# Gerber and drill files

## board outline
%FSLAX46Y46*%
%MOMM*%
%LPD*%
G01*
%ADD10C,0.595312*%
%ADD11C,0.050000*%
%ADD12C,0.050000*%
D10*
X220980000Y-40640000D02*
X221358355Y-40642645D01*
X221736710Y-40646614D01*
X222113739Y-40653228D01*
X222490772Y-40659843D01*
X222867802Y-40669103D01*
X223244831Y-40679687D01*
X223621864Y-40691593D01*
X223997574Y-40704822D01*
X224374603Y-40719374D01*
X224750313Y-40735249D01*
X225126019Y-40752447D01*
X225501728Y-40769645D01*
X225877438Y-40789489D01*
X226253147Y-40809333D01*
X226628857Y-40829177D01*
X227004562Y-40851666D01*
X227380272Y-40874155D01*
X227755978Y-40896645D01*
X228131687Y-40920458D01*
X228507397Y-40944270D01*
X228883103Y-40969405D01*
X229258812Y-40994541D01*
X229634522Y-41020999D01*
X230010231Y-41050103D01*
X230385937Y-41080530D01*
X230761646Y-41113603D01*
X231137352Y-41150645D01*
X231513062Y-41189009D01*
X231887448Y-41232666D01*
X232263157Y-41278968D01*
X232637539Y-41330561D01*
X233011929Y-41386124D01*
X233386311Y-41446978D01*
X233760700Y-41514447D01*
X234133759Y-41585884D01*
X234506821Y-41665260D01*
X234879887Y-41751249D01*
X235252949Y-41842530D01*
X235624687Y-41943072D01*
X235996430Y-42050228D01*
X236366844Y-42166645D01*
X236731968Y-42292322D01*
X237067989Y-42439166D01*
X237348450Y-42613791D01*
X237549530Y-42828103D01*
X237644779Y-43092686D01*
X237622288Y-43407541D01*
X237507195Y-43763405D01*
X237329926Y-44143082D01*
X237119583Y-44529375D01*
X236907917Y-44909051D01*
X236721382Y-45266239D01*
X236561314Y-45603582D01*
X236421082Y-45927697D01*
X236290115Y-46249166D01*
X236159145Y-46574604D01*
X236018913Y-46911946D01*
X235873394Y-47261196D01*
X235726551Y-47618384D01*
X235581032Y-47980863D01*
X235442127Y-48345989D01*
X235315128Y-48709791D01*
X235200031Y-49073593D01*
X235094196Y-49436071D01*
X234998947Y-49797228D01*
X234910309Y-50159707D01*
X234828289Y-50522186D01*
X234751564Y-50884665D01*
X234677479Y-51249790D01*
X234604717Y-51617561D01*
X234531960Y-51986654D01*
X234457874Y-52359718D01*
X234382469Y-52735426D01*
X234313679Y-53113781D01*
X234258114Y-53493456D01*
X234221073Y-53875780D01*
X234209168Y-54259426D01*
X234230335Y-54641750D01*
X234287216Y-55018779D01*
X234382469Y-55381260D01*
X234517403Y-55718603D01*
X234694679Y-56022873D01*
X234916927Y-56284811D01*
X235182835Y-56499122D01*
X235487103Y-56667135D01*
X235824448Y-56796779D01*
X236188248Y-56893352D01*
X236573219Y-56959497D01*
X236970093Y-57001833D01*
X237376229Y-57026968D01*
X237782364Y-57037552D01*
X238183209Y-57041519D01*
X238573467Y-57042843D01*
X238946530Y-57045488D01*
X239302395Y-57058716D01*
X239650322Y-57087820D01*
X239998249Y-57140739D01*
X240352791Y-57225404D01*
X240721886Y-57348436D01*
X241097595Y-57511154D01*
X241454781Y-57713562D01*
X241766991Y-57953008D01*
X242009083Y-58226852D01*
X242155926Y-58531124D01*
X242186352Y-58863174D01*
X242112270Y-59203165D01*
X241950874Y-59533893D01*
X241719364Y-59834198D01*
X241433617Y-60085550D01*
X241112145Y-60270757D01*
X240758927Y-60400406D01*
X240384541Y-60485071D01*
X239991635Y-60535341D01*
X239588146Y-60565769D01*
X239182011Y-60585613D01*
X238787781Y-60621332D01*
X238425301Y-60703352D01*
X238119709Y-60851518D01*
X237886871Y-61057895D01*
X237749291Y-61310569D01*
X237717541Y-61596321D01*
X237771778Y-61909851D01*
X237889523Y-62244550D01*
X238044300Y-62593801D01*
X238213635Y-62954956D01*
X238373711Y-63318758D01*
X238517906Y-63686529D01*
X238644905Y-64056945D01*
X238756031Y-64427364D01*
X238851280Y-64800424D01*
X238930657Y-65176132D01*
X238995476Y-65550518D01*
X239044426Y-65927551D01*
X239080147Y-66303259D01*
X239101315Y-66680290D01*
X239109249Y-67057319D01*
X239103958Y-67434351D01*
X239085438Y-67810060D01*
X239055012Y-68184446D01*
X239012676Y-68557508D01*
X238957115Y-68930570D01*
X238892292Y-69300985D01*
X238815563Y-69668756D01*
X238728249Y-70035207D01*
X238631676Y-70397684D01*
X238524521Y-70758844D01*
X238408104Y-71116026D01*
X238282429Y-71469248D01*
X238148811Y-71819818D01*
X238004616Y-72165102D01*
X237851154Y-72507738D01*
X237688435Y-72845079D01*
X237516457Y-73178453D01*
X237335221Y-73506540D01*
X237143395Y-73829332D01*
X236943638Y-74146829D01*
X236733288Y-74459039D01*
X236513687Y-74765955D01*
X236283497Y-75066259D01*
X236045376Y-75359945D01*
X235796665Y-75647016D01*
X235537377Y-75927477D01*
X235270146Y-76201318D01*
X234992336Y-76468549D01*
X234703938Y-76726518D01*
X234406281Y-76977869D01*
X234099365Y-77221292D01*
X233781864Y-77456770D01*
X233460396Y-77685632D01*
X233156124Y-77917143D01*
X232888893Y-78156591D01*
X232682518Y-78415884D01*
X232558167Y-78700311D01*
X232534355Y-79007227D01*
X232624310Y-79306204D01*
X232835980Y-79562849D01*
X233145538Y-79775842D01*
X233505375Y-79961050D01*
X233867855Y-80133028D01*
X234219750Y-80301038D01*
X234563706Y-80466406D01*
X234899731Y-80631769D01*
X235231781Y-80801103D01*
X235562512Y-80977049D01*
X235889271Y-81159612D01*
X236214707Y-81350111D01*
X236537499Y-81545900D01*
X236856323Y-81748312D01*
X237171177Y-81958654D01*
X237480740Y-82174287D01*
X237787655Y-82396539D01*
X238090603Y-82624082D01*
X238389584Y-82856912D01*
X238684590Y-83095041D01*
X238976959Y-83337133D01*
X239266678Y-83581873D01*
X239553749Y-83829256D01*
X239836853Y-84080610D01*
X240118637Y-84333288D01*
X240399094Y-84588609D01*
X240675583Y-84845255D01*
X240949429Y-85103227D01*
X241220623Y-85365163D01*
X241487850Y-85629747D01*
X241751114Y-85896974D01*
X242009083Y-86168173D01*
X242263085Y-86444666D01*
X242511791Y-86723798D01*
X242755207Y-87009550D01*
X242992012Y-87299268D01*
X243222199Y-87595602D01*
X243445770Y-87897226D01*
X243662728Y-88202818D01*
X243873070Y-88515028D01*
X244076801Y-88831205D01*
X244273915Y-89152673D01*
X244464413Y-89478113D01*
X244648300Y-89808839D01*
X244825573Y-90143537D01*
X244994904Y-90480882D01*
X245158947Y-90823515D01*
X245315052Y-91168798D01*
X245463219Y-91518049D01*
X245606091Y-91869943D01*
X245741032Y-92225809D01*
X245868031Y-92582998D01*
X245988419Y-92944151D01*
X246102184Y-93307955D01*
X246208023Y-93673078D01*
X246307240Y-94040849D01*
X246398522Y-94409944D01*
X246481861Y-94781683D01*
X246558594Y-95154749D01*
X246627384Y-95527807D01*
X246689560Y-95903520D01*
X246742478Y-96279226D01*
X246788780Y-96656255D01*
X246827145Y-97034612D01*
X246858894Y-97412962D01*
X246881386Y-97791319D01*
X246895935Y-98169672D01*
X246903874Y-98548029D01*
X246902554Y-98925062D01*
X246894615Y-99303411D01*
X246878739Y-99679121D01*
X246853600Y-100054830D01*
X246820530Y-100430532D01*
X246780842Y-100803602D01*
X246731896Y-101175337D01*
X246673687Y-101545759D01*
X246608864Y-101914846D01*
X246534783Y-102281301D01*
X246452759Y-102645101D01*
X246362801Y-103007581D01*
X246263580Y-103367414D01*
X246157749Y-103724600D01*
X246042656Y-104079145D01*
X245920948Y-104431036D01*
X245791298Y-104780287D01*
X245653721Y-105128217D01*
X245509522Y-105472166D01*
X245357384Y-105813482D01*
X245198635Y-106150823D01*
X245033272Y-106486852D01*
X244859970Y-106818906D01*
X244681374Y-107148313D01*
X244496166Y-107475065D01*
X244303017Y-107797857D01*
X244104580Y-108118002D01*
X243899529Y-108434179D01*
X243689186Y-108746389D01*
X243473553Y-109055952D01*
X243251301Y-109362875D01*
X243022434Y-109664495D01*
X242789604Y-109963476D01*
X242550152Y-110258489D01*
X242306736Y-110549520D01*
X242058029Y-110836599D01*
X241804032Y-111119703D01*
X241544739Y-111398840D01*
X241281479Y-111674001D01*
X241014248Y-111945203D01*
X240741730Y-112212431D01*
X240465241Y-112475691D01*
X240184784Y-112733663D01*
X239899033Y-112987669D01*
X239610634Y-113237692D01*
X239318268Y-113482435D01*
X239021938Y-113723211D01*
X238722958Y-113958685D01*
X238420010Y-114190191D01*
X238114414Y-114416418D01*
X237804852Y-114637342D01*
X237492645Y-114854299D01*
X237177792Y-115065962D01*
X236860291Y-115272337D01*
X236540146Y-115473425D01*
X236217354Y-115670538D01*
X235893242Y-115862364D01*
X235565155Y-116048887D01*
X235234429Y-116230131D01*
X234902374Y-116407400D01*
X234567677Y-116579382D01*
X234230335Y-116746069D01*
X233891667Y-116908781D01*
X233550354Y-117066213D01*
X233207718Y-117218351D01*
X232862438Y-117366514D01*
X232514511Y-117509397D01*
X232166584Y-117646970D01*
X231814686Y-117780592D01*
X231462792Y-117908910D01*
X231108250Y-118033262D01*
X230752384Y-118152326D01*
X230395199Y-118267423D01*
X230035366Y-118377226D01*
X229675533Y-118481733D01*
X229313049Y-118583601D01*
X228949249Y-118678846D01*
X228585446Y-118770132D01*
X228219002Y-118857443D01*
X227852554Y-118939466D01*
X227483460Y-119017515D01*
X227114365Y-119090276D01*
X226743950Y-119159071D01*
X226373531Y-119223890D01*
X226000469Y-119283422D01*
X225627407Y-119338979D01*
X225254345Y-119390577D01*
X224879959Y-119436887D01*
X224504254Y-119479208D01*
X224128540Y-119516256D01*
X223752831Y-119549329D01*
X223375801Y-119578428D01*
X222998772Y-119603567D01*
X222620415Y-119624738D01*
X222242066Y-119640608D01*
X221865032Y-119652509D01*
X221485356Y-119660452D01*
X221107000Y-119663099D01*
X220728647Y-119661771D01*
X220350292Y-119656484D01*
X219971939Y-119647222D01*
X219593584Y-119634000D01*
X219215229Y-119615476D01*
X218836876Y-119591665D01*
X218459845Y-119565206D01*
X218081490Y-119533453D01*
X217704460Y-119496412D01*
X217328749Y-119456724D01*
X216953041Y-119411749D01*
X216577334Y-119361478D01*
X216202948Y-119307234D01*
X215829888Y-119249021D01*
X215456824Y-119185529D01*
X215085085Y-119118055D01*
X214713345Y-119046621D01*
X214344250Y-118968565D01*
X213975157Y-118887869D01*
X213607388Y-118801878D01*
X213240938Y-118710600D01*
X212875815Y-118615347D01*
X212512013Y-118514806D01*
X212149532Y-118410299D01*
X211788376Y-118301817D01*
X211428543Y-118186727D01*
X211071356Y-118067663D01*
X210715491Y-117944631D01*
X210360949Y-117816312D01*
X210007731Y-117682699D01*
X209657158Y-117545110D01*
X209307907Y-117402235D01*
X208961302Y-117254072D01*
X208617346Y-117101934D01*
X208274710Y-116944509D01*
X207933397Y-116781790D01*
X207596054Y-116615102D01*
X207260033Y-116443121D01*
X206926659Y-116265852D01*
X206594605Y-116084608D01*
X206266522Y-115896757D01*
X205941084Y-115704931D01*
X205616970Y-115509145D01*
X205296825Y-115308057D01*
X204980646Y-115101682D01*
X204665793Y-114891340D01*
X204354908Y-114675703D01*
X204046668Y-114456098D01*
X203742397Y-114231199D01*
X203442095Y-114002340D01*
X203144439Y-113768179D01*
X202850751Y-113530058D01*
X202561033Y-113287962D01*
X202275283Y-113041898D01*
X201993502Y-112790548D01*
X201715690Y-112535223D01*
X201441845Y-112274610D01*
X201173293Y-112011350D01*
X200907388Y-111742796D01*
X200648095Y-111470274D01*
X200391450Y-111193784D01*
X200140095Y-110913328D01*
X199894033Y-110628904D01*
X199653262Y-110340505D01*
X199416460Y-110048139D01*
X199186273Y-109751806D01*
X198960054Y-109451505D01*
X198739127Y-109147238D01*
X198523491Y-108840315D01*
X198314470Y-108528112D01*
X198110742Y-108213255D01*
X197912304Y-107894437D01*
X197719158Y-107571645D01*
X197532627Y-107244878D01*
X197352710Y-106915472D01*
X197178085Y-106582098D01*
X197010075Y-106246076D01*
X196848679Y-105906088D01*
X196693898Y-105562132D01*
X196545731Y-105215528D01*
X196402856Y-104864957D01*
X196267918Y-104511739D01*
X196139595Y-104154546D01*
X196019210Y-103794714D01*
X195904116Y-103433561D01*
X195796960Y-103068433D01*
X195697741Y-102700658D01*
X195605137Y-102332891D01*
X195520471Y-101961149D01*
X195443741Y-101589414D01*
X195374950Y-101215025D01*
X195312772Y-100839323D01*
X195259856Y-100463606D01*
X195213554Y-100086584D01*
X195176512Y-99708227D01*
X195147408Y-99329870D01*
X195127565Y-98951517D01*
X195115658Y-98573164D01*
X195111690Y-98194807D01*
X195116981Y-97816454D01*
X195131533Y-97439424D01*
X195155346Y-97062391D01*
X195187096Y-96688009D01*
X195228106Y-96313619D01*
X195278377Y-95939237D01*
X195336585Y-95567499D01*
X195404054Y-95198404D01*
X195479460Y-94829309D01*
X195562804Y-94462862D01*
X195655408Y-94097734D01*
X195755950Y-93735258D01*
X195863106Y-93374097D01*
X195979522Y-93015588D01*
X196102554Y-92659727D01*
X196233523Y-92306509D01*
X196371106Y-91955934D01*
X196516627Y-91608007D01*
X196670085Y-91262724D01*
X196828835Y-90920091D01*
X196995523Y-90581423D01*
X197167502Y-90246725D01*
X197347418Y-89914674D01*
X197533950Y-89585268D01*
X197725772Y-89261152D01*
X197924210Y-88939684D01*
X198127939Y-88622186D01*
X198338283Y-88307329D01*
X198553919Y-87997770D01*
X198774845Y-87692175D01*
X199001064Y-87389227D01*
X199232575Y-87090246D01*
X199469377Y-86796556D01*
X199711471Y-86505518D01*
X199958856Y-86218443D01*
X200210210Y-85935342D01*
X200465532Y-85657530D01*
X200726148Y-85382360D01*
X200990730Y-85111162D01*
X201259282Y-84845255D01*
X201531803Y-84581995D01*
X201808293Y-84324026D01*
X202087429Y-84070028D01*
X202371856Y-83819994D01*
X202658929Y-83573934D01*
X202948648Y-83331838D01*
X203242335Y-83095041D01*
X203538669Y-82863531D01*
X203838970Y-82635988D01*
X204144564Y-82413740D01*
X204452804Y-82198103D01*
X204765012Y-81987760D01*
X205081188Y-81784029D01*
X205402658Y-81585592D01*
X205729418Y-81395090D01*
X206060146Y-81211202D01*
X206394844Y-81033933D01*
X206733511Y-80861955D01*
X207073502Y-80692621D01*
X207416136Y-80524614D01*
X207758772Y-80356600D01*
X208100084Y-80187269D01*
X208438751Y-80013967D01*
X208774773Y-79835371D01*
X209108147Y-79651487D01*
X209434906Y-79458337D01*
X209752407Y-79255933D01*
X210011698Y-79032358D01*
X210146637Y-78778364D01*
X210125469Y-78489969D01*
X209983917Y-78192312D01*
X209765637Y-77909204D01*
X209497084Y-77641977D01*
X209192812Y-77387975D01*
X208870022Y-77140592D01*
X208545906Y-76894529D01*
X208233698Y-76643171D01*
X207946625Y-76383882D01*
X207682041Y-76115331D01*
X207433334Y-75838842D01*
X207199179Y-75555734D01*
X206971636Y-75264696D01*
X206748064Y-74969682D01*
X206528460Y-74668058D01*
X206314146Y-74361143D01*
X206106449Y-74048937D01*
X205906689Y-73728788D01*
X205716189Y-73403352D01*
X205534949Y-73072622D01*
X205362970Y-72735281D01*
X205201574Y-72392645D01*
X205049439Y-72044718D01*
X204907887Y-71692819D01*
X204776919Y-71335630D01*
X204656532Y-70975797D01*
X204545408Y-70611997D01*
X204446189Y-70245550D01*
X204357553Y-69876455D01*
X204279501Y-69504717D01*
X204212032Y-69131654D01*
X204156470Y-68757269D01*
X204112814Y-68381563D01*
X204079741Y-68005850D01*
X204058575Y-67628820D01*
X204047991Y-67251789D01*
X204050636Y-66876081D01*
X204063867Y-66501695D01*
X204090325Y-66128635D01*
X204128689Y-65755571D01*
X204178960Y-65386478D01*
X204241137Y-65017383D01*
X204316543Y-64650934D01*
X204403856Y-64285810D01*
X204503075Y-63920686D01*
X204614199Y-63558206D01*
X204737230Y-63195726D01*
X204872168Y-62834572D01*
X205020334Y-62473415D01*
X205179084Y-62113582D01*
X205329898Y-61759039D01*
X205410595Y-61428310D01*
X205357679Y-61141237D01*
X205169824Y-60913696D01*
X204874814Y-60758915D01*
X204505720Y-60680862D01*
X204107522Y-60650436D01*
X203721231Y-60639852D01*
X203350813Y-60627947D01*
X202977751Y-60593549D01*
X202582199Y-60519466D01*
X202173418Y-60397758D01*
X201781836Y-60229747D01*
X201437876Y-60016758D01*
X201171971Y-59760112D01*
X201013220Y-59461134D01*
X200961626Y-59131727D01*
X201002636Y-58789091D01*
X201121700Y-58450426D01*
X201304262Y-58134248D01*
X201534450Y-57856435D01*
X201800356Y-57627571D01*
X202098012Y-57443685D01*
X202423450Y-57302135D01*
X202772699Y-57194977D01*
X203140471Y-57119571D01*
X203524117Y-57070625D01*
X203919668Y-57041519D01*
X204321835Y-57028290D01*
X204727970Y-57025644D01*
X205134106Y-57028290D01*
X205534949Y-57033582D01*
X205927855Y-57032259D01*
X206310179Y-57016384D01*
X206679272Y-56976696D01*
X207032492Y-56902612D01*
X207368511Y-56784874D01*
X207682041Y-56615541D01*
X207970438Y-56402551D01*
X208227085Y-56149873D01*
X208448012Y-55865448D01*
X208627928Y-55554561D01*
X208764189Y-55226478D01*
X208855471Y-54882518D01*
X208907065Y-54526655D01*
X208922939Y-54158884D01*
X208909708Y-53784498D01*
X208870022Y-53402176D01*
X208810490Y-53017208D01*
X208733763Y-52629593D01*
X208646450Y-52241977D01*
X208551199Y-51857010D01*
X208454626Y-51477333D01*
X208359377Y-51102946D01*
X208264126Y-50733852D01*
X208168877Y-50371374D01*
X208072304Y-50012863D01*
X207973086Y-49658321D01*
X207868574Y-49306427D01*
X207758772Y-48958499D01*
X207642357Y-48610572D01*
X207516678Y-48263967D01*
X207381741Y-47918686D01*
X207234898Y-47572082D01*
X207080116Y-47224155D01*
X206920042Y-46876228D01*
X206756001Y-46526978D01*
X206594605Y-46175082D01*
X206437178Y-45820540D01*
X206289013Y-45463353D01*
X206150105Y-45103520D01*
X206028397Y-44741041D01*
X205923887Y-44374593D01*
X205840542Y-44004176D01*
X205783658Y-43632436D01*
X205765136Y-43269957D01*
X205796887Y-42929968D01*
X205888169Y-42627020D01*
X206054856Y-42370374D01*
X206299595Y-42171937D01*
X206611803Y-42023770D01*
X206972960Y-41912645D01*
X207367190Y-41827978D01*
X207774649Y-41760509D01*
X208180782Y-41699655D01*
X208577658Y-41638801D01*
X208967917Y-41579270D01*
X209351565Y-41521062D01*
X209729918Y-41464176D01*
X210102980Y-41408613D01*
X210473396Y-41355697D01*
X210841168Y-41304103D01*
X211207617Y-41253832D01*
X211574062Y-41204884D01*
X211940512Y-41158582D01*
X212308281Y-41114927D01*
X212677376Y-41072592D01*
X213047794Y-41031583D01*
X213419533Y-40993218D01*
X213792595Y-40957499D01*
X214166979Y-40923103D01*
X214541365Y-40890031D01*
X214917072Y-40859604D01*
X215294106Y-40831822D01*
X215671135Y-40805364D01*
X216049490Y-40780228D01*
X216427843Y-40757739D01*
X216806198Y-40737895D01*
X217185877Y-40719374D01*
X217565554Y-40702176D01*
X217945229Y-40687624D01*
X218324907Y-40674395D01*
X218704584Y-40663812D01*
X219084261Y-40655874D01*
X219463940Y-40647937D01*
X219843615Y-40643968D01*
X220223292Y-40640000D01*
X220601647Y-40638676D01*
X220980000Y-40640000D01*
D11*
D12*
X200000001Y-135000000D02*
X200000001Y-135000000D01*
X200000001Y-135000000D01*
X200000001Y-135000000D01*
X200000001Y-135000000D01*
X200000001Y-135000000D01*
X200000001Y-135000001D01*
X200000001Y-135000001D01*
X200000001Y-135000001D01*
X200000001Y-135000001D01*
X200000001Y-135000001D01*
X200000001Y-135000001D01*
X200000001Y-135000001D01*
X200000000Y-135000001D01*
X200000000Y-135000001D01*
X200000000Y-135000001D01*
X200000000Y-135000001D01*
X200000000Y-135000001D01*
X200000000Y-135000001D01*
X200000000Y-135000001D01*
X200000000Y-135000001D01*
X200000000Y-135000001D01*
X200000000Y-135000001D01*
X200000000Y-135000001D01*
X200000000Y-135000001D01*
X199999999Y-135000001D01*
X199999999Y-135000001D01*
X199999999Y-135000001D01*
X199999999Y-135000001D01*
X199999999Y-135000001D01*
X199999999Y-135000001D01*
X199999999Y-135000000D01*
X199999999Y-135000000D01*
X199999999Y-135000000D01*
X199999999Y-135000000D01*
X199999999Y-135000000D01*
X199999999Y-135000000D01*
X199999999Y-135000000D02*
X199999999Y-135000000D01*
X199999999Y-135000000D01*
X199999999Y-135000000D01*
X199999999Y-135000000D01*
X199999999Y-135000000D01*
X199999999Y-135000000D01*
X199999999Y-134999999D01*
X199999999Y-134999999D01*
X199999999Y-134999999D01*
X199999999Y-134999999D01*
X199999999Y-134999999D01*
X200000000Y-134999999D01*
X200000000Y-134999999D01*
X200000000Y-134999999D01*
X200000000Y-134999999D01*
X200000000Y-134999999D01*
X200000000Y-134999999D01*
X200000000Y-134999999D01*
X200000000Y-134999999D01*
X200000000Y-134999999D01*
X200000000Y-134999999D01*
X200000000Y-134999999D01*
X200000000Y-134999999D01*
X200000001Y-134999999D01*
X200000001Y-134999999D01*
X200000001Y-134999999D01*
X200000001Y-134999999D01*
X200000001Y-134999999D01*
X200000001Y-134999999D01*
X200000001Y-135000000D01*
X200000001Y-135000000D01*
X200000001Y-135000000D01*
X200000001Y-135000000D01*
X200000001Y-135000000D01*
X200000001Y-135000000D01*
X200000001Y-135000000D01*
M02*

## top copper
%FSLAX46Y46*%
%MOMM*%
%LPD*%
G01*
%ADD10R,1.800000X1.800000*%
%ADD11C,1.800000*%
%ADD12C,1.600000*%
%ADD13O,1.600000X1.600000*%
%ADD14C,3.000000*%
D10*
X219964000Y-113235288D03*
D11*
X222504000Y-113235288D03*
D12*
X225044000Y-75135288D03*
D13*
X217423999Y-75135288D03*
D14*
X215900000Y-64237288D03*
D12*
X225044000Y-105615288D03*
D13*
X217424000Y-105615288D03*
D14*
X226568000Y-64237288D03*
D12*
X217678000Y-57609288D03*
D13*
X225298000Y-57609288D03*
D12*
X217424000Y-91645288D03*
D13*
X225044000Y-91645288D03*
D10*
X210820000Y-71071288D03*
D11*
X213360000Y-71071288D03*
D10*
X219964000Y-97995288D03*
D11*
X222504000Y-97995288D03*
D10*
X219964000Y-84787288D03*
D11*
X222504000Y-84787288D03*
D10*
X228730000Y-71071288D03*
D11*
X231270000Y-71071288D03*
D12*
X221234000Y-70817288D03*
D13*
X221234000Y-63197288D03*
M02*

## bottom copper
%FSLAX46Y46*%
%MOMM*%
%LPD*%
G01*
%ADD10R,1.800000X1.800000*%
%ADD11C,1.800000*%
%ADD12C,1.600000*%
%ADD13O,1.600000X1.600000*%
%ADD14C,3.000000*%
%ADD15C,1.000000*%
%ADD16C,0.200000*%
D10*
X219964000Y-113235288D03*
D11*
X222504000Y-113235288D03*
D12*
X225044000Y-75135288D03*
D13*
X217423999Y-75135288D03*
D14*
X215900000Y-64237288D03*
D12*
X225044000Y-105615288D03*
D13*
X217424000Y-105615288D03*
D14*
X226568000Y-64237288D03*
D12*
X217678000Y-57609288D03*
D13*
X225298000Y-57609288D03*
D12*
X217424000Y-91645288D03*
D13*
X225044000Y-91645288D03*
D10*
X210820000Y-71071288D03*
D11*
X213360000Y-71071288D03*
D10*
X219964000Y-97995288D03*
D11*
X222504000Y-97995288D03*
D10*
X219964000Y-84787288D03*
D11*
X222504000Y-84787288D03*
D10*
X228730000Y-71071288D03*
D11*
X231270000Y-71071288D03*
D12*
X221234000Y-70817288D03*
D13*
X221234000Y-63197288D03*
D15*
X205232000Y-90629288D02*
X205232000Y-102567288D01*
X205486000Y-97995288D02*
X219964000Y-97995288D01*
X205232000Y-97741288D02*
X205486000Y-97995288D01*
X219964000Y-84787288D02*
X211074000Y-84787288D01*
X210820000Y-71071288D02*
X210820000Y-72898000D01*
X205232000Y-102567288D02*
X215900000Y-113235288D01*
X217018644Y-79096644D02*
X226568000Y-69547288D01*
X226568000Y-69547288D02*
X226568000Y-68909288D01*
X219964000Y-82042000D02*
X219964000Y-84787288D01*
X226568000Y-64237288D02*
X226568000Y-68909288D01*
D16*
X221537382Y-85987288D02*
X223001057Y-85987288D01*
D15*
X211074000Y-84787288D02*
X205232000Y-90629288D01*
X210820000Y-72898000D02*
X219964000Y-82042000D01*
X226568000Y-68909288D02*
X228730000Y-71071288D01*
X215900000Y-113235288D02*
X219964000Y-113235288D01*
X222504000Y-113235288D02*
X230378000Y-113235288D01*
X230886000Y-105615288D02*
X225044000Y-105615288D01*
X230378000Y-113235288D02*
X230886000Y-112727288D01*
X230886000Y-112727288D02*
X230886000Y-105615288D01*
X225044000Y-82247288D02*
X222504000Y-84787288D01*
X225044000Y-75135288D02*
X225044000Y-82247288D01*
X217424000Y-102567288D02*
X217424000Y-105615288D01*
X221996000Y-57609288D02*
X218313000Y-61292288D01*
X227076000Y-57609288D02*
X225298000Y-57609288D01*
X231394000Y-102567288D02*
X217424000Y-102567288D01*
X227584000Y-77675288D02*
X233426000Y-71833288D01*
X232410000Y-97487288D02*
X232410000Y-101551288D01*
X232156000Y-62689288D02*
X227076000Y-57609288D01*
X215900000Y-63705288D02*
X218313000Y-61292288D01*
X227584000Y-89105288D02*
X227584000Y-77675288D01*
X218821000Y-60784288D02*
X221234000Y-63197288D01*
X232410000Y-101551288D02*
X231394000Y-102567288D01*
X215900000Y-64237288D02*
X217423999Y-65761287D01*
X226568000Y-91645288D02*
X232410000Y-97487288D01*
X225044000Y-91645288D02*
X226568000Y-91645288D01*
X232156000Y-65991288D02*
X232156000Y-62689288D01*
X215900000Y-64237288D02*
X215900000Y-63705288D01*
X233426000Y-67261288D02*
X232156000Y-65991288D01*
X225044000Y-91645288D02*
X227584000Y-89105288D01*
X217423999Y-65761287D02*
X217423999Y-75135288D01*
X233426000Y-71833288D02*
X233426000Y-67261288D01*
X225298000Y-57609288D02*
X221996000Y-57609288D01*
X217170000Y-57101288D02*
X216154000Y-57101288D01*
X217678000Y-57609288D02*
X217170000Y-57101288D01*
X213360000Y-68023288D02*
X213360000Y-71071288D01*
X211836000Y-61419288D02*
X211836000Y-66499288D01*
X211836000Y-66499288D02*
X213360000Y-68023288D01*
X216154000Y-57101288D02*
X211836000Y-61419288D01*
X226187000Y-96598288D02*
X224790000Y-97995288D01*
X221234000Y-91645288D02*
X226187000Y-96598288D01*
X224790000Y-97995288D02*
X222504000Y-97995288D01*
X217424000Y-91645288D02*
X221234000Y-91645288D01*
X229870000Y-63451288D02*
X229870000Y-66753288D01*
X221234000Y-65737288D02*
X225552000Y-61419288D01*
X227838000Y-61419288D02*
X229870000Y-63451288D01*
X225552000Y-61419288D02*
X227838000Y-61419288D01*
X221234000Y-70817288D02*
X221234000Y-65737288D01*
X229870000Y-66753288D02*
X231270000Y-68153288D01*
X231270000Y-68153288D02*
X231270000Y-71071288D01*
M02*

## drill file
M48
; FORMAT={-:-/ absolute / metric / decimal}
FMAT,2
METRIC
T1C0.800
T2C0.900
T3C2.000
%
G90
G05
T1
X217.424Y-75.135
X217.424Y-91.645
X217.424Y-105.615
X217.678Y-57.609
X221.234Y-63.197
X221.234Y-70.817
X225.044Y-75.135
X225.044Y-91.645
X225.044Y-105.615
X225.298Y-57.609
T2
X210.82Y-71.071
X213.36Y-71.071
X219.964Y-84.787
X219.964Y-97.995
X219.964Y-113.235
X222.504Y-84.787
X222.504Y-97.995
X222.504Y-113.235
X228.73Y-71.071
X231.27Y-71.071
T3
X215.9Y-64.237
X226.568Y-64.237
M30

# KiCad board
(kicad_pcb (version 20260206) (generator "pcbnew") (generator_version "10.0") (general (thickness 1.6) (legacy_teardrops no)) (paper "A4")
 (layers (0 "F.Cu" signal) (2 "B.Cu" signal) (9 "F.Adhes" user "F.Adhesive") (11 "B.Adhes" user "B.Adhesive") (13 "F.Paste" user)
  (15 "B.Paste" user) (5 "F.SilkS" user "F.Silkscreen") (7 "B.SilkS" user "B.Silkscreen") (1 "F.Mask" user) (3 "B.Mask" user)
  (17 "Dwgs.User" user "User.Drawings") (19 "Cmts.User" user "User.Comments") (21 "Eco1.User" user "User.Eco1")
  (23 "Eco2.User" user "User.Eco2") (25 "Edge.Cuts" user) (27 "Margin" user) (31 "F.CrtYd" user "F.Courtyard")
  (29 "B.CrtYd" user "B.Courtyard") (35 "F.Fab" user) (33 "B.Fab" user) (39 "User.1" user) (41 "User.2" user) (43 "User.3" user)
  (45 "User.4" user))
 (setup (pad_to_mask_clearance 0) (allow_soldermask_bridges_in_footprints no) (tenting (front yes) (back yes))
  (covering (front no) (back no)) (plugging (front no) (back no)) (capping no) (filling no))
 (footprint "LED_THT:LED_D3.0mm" (layer "F.Cu") (at 219.964 113.235288)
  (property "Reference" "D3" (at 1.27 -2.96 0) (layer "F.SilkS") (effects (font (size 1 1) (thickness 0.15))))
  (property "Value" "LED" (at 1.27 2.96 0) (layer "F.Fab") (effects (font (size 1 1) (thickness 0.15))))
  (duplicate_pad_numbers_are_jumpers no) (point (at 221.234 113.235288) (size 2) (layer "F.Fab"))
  (pad "1" thru_hole rect (at 0 0) (size 1.8 1.8) (drill 0.9) (layers "*.Cu" "*.Mask") (remove_unused_layers no) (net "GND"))
  (pad "2" thru_hole circle (at 2.54 0) (size 1.8 1.8) (drill 0.9) (layers "*.Cu" "*.Mask") (remove_unused_layers no) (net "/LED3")))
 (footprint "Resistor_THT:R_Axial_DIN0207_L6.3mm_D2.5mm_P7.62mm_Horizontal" (layer "F.Cu") (at 225.044 75.135288 180)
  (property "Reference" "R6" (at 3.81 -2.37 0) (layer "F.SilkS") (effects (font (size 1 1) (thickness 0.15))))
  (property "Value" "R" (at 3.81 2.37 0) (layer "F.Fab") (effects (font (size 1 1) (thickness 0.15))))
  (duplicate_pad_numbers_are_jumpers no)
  (pad "1" thru_hole circle (at 0 0 180) (size 1.6 1.6) (drill 0.8) (layers "*.Cu" "*.Mask") (remove_unused_layers no) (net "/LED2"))
  (pad "2" thru_hole oval (at 7.620001 0 180) (size 1.6 1.6) (drill 0.8) (layers "*.Cu" "*.Mask") (remove_unused_layers no) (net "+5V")))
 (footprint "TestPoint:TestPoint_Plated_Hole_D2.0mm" (layer "F.Cu") (at 215.9 64.237288)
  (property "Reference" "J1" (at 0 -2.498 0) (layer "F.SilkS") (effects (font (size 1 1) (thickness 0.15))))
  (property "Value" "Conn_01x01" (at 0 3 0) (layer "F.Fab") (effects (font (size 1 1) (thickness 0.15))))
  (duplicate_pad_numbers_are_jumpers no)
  (pad "1" thru_hole circle (at 0 0) (size 3 3) (drill 2) (layers "*.Cu" "*.Mask") (remove_unused_layers no) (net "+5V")))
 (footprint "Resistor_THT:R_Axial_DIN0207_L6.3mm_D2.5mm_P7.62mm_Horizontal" (layer "F.Cu") (at 225.044 105.615288 180)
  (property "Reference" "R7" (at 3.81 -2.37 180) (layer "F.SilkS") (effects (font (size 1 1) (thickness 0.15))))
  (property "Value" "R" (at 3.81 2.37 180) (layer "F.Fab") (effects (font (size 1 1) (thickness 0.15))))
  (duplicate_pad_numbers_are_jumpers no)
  (pad "1" thru_hole circle (at 0 0 180) (size 1.6 1.6) (drill 0.8) (layers "*.Cu" "*.Mask") (remove_unused_layers no) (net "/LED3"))
  (pad "2" thru_hole oval (at 7.62 0 180) (size 1.6 1.6) (drill 0.8) (layers "*.Cu" "*.Mask") (remove_unused_layers no) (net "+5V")))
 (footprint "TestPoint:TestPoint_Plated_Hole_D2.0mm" (layer "F.Cu") (at 226.568 64.237288)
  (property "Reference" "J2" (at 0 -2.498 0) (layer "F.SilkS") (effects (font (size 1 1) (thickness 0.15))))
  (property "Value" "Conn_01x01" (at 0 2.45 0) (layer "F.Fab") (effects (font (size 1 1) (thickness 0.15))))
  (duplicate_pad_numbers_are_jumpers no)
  (pad "1" thru_hole circle (at 0 0) (size 3 3) (drill 2) (layers "*.Cu" "*.Mask") (remove_unused_layers no) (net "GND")))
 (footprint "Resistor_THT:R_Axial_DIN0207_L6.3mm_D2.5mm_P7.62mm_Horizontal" (layer "F.Cu") (at 217.678 57.609288)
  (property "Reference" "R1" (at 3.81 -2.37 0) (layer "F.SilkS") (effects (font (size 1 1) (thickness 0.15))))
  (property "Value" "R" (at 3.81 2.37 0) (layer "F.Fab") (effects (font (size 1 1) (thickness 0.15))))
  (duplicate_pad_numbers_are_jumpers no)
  (pad "1" thru_hole circle (at 0 0) (size 1.6 1.6) (drill 0.8) (layers "*.Cu" "*.Mask") (remove_unused_layers no) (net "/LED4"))
  (pad "2" thru_hole oval (at 7.62 0) (size 1.6 1.6) (drill 0.8) (layers "*.Cu" "*.Mask") (remove_unused_layers no) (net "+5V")))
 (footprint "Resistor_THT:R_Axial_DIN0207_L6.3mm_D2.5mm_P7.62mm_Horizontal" (layer "F.Cu") (at 217.424 91.645288)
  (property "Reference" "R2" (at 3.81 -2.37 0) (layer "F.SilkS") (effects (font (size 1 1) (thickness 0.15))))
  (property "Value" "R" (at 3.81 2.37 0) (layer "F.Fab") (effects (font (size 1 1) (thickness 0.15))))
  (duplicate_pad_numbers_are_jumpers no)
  (pad "1" thru_hole circle (at 0 0) (size 1.6 1.6) (drill 0.8) (layers "*.Cu" "*.Mask") (remove_unused_layers no) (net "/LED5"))
  (pad "2" thru_hole oval (at 7.62 0) (size 1.6 1.6) (drill 0.8) (layers "*.Cu" "*.Mask") (remove_unused_layers no) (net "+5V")))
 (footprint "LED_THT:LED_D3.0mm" (layer "F.Cu") (at 210.82 71.071288)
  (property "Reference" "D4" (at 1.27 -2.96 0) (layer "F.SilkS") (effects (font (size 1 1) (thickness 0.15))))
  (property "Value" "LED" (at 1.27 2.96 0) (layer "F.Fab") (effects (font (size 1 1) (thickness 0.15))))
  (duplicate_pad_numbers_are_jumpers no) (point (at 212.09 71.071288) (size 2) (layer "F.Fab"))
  (pad "1" thru_hole rect (at 0 0) (size 1.8 1.8) (drill 0.9) (layers "*.Cu" "*.Mask") (remove_unused_layers no) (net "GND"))
  (pad "2" thru_hole circle (at 2.54 0) (size 1.8 1.8) (drill 0.9) (layers "*.Cu" "*.Mask") (remove_unused_layers no) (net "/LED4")))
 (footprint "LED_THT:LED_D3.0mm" (layer "F.Cu") (at 219.964 97.995288)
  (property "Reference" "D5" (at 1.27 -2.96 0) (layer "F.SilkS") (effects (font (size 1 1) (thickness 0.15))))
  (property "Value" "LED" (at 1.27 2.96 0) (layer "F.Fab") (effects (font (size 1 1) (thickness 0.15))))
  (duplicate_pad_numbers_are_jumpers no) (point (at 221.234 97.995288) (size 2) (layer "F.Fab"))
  (pad "1" thru_hole rect (at 0 0) (size 1.8 1.8) (drill 0.9) (layers "*.Cu" "*.Mask") (remove_unused_layers no) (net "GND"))
  (pad "2" thru_hole circle (at 2.54 0) (size 1.8 1.8) (drill 0.9) (layers "*.Cu" "*.Mask") (remove_unused_layers no) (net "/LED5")))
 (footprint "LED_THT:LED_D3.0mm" (layer "F.Cu") (at 219.964 84.787288)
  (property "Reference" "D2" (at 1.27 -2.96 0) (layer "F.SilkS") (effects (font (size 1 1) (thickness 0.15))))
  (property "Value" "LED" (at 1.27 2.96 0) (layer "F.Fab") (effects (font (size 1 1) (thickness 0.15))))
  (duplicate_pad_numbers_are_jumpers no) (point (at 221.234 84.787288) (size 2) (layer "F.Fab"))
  (pad "1" thru_hole rect (at 0 0) (size 1.8 1.8) (drill 0.9) (layers "*.Cu" "*.Mask") (remove_unused_layers no) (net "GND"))
  (pad "2" thru_hole circle (at 2.54 0) (size 1.8 1.8) (drill 0.9) (layers "*.Cu" "*.Mask") (remove_unused_layers no) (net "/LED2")))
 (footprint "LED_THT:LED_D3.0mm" (layer "F.Cu") (at 228.73 71.071288)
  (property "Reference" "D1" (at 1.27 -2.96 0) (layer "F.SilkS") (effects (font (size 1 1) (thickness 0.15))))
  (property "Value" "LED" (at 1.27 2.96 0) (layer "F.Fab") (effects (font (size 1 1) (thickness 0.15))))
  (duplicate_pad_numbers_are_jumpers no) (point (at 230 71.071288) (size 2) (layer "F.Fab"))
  (pad "1" thru_hole rect (at 0 0) (size 1.8 1.8) (drill 0.9) (layers "*.Cu" "*.Mask") (remove_unused_layers no) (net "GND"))
  (pad "2" thru_hole circle (at 2.54 0) (size 1.8 1.8) (drill 0.9) (layers "*.Cu" "*.Mask") (remove_unused_layers no) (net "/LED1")))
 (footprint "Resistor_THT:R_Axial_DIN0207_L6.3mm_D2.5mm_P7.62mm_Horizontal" (layer "F.Cu") (at 221.234 70.817288 90)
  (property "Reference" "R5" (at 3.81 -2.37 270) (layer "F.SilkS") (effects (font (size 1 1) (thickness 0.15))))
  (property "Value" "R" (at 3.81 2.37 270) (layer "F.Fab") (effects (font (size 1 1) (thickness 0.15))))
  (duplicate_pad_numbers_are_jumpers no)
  (pad "1" thru_hole circle (at 0 0 90) (size 1.6 1.6) (drill 0.8) (layers "*.Cu" "*.Mask") (remove_unused_layers no) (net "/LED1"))
  (pad "2" thru_hole oval (at 7.62 0 90) (size 1.6 1.6) (drill 0.8) (layers "*.Cu" "*.Mask") (remove_unused_layers no) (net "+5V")))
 (gr_poly
  (pts (xy 220.98 40.64) (xy 221.358355 40.642645) (xy 221.73671 40.646614) (xy 222.113739 40.653228) (xy 222.490772 40.659843)
   (xy 222.867802 40.669103) (xy 223.244831 40.679687) (xy 223.621864 40.691593) (xy 223.997574 40.704822) (xy 224.374603 40.719374)
   (xy 224.750313 40.735249) (xy 225.126019 40.752447) (xy 225.501728 40.769645) (xy 225.877438 40.789489) (xy 226.253147 40.809333)
   (xy 226.628857 40.829177) (xy 227.004562 40.851666) (xy 227.380272 40.874155) (xy 227.755978 40.896645) (xy 228.131687 40.920458)
   (xy 228.507397 40.94427) (xy 228.883103 40.969405) (xy 229.258812 40.994541) (xy 229.634522 41.020999) (xy 230.010231 41.050103)
   (xy 230.385937 41.08053) (xy 230.761646 41.113603) (xy 231.137352 41.150645) (xy 231.513062 41.189009) (xy 231.887448 41.232666)
   (xy 232.263157 41.278968) (xy 232.637539 41.330561) (xy 233.011929 41.386124) (xy 233.386311 41.446978) (xy 233.7607 41.514447)
   (xy 234.133759 41.585884) (xy 234.506821 41.66526) (xy 234.879887 41.751249) (xy 235.252949 41.84253) (xy 235.624687 41.943072)
   (xy 235.99643 42.050228) (xy 236.366844 42.166645) (xy 236.731968 42.292322) (xy 237.067989 42.439166) (xy 237.34845 42.613791)
   (xy 237.54953 42.828103) (xy 237.644779 43.092686) (xy 237.622288 43.407541) (xy 237.507195 43.763405) (xy 237.329926 44.143082)
   (xy 237.119583 44.529375) (xy 236.907917 44.909051) (xy 236.721382 45.266239) (xy 236.561314 45.603582) (xy 236.421082 45.927697)
   (xy 236.290115 46.249166) (xy 236.159145 46.574604) (xy 236.018913 46.911946) (xy 235.873394 47.261196) (xy 235.726551 47.618384)
   (xy 235.581032 47.980863) (xy 235.442127 48.345989) (xy 235.315128 48.709791) (xy 235.200031 49.073593) (xy 235.094196 49.436071)
   (xy 234.998947 49.797228) (xy 234.910309 50.159707) (xy 234.828289 50.522186) (xy 234.751564 50.884665) (xy 234.677479 51.24979)
   (xy 234.604717 51.617561) (xy 234.53196 51.986654) (xy 234.457874 52.359718) (xy 234.382469 52.735426) (xy 234.313679 53.113781)
   (xy 234.258114 53.493456) (xy 234.221073 53.87578) (xy 234.209168 54.259426) (xy 234.230335 54.64175) (xy 234.287216 55.018779)
   (xy 234.382469 55.38126) (xy 234.517403 55.718603) (xy 234.694679 56.022873) (xy 234.916927 56.284811) (xy 235.182835 56.499122)
   (xy 235.487103 56.667135) (xy 235.824448 56.796779) (xy 236.188248 56.893352) (xy 236.573219 56.959497) (xy 236.970093 57.001833)
   (xy 237.376229 57.026968) (xy 237.782364 57.037552) (xy 238.183209 57.041519) (xy 238.573467 57.042843) (xy 238.94653 57.045488)
   (xy 239.302395 57.058716) (xy 239.650322 57.08782) (xy 239.998249 57.140739) (xy 240.352791 57.225404) (xy 240.721886 57.348436)
   (xy 241.097595 57.511154) (xy 241.454781 57.713562) (xy 241.766991 57.953008) (xy 242.009083 58.226852) (xy 242.155926 58.531124)
   (xy 242.186352 58.863174) (xy 242.11227 59.203165) (xy 241.950874 59.533893) (xy 241.719364 59.834198) (xy 241.433617 60.08555)
   (xy 241.112145 60.270757) (xy 240.758927 60.400406) (xy 240.384541 60.485071) (xy 239.991635 60.535341) (xy 239.588146 60.565769)
   (xy 239.182011 60.585613) (xy 238.787781 60.621332) (xy 238.425301 60.703352) (xy 238.119709 60.851518) (xy 237.886871 61.057895)
   (xy 237.749291 61.310569) (xy 237.717541 61.596321) (xy 237.771778 61.909851) (xy 237.889523 62.24455) (xy 238.0443 62.593801)
   (xy 238.213635 62.954956) (xy 238.373711 63.318758) (xy 238.517906 63.686529) (xy 238.644905 64.056945) (xy 238.756031 64.427364)
   (xy 238.85128 64.800424) (xy 238.930657 65.176132) (xy 238.995476 65.550518) (xy 239.044426 65.927551) (xy 239.080147 66.303259)
   (xy 239.101315 66.68029) (xy 239.109249 67.057319) (xy 239.103958 67.434351) (xy 239.085438 67.81006) (xy 239.055012 68.184446)
   (xy 239.012676 68.557508) (xy 238.957115 68.93057) (xy 238.892292 69.300985) (xy 238.815563 69.668756) (xy 238.728249 70.035207)
   (xy 238.631676 70.397684) (xy 238.524521 70.758844) (xy 238.408104 71.116026) (xy 238.282429 71.469248) (xy 238.148811 71.819818)
   (xy 238.004616 72.165102) (xy 237.851154 72.507738) (xy 237.688435 72.845079) (xy 237.516457 73.178453) (xy 237.335221 73.50654)
   (xy 237.143395 73.829332) (xy 236.943638 74.146829) (xy 236.733288 74.459039) (xy 236.513687 74.765955) (xy 236.283497 75.066259)
   (xy 236.045376 75.359945) (xy 235.796665 75.647016) (xy 235.537377 75.927477) (xy 235.270146 76.201318) (xy 234.992336 76.468549)
   (xy 234.703938 76.726518) (xy 234.406281 76.977869) (xy 234.099365 77.221292) (xy 233.781864 77.45677) (xy 233.460396 77.685632)
   (xy 233.156124 77.917143) (xy 232.888893 78.156591) (xy 232.682518 78.415884) (xy 232.558167 78.700311) (xy 232.534355 79.007227)
   (xy 232.62431 79.306204) (xy 232.83598 79.562849) (xy 233.145538 79.775842) (xy 233.505375 79.96105) (xy 233.867855 80.133028)
   (xy 234.21975 80.301038) (xy 234.563706 80.466406) (xy 234.899731 80.631769) (xy 235.231781 80.801103) (xy 235.562512 80.977049)
   (xy 235.889271 81.159612) (xy 236.214707 81.350111) (xy 236.537499 81.5459) (xy 236.856323 81.748312) (xy 237.171177 81.958654)
   (xy 237.48074 82.174287) (xy 237.787655 82.396539) (xy 238.090603 82.624082) (xy 238.389584 82.856912) (xy 238.68459 83.095041)
   (xy 238.976959 83.337133) (xy 239.266678 83.581873) (xy 239.553749 83.829256) (xy 239.836853 84.08061) (xy 240.118637 84.333288)
   (xy 240.399094 84.588609) (xy 240.675583 84.845255) (xy 240.949429 85.103227) (xy 241.220623 85.365163) (xy 241.48785 85.629747)
   (xy 241.751114 85.896974) (xy 242.009083 86.168173) (xy 242.263085 86.444666) (xy 242.511791 86.723798) (xy 242.755207 87.00955)
   (xy 242.992012 87.299268) (xy 243.222199 87.595602) (xy 243.44577 87.897226) (xy 243.662728 88.202818) (xy 243.87307 88.515028)
   (xy 244.076801 88.831205) (xy 244.273915 89.152673) (xy 244.464413 89.478113) (xy 244.6483 89.808839) (xy 244.825573 90.143537)
   (xy 244.994904 90.480882) (xy 245.158947 90.823515) (xy 245.315052 91.168798) (xy 245.463219 91.518049) (xy 245.606091 91.869943)
   (xy 245.741032 92.225809) (xy 245.868031 92.582998) (xy 245.988419 92.944151) (xy 246.102184 93.307955) (xy 246.208023 93.673078)
   (xy 246.30724 94.040849) (xy 246.398522 94.409944) (xy 246.481861 94.781683) (xy 246.558594 95.154749) (xy 246.627384 95.527807)
   (xy 246.68956 95.90352) (xy 246.742478 96.279226) (xy 246.78878 96.656255) (xy 246.827145 97.034612) (xy 246.858894 97.412962)
   (xy 246.881386 97.791319) (xy 246.895935 98.169672) (xy 246.903874 98.548029) (xy 246.902554 98.925062) (xy 246.894615 99.303411)
   (xy 246.878739 99.679121) (xy 246.8536 100.05483) (xy 246.82053 100.430532) (xy 246.780842 100.803602) (xy 246.731896 101.175337)
   (xy 246.673687 101.545759) (xy 246.608864 101.914846) (xy 246.534783 102.281301) (xy 246.452759 102.645101) (xy 246.362801 103.007581)
   (xy 246.26358 103.367414) (xy 246.157749 103.7246) (xy 246.042656 104.079145) (xy 245.920948 104.431036) (xy 245.791298 104.780287)
   (xy 245.653721 105.128217) (xy 245.509522 105.472166) (xy 245.357384 105.813482) (xy 245.198635 106.150823) (xy 245.033272 106.486852)
   (xy 244.85997 106.818906) (xy 244.681374 107.148313) (xy 244.496166 107.475065) (xy 244.303017 107.797857) (xy 244.10458 108.118002)
   (xy 243.899529 108.434179) (xy 243.689186 108.746389) (xy 243.473553 109.055952) (xy 243.251301 109.362875) (xy 243.022434 109.664495)
   (xy 242.789604 109.963476) (xy 242.550152 110.258489) (xy 242.306736 110.54952) (xy 242.058029 110.836599) (xy 241.804032 111.119703)
   (xy 241.544739 111.39884) (xy 241.281479 111.674001) (xy 241.014248 111.945203) (xy 240.74173 112.212431) (xy 240.465241 112.475691)
   (xy 240.184784 112.733663) (xy 239.899033 112.987669) (xy 239.610634 113.237692) (xy 239.318268 113.482435) (xy 239.021938 113.723211)
   (xy 238.722958 113.958685) (xy 238.42001 114.190191) (xy 238.114414 114.416418) (xy 237.804852 114.637342) (xy 237.492645 114.854299)
   (xy 237.177792 115.065962) (xy 236.860291 115.272337) (xy 236.540146 115.473425) (xy 236.217354 115.670538) (xy 235.893242 115.862364)
   (xy 235.565155 116.048887) (xy 235.234429 116.230131) (xy 234.902374 116.4074) (xy 234.567677 116.579382) (xy 234.230335 116.746069)
   (xy 233.891667 116.908781) (xy 233.550354 117.066213) (xy 233.207718 117.218351) (xy 232.862438 117.366514) (xy 232.514511 117.509397)
   (xy 232.166584 117.64697) (xy 231.814686 117.780592) (xy 231.462792 117.90891) (xy 231.10825 118.033262) (xy 230.752384 118.152326)
   (xy 230.395199 118.267423) (xy 230.035366 118.377226) (xy 229.675533 118.481733) (xy 229.313049 118.583601) (xy 228.949249 118.678846)
   (xy 228.585446 118.770132) (xy 228.219002 118.857443) (xy 227.852554 118.939466) (xy 227.48346 119.017515) (xy 227.114365 119.090276)
   (xy 226.74395 119.159071) (xy 226.373531 119.22389) (xy 226.000469 119.283422) (xy 225.627407 119.338979) (xy 225.254345 119.390577)
   (xy 224.879959 119.436887) (xy 224.504254 119.479208) (xy 224.12854 119.516256) (xy 223.752831 119.549329) (xy 223.375801 119.578428)
   (xy 222.998772 119.603567) (xy 222.620415 119.624738) (xy 222.242066 119.640608) (xy 221.865032 119.652509) (xy 221.485356 119.660452)
   (xy 221.107 119.663099) (xy 220.728647 119.661771) (xy 220.350292 119.656484) (xy 219.971939 119.647222) (xy 219.593584 119.634)
   (xy 219.215229 119.615476) (xy 218.836876 119.591665) (xy 218.459845 119.565206) (xy 218.08149 119.533453) (xy 217.70446 119.496412)
   (xy 217.328749 119.456724) (xy 216.953041 119.411749) (xy 216.577334 119.361478) (xy 216.202948 119.307234) (xy 215.829888 119.249021)
   (xy 215.456824 119.185529) (xy 215.085085 119.118055) (xy 214.713345 119.046621) (xy 214.34425 118.968565) (xy 213.975157 118.887869)
   (xy 213.607388 118.801878) (xy 213.240938 118.7106) (xy 212.875815 118.615347) (xy 212.512013 118.514806) (xy 212.149532 118.410299)
   (xy 211.788376 118.301817) (xy 211.428543 118.186727) (xy 211.071356 118.067663) (xy 210.715491 117.944631) (xy 210.360949 117.816312)
   (xy 210.007731 117.682699) (xy 209.657158 117.54511) (xy 209.307907 117.402235) (xy 208.961302 117.254072) (xy 208.617346 117.101934)
   (xy 208.27471 116.944509) (xy 207.933397 116.78179) (xy 207.596054 116.615102) (xy 207.260033 116.443121) (xy 206.926659 116.265852)
   (xy 206.594605 116.084608) (xy 206.266522 115.896757) (xy 205.941084 115.704931) (xy 205.61697 115.509145) (xy 205.296825 115.308057)
   (xy 204.980646 115.101682) (xy 204.665793 114.89134) (xy 204.354908 114.675703) (xy 204.046668 114.456098) (xy 203.742397 114.231199)
   (xy 203.442095 114.00234) (xy 203.144439 113.768179) (xy 202.850751 113.530058) (xy 202.561033 113.287962) (xy 202.275283 113.041898)
   (xy 201.993502 112.790548) (xy 201.71569 112.535223) (xy 201.441845 112.27461) (xy 201.173293 112.01135) (xy 200.907388 111.742796)
   (xy 200.648095 111.470274) (xy 200.39145 111.193784) (xy 200.140095 110.913328) (xy 199.894033 110.628904) (xy 199.653262 110.340505)
   (xy 199.41646 110.048139) (xy 199.186273 109.751806) (xy 198.960054 109.451505) (xy 198.739127 109.147238) (xy 198.523491 108.840315)
   (xy 198.31447 108.528112) (xy 198.110742 108.213255) (xy 197.912304 107.894437) (xy 197.719158 107.571645) (xy 197.532627 107.244878)
   (xy 197.35271 106.915472) (xy 197.178085 106.582098) (xy 197.010075 106.246076) (xy 196.848679 105.906088) (xy 196.693898 105.562132)
   (xy 196.545731 105.215528) (xy 196.402856 104.864957) (xy 196.267918 104.511739) (xy 196.139595 104.154546) (xy 196.01921 103.794714)
   (xy 195.904116 103.433561) (xy 195.79696 103.068433) (xy 195.697741 102.700658) (xy 195.605137 102.332891) (xy 195.520471 101.961149)
   (xy 195.443741 101.589414) (xy 195.37495 101.215025) (xy 195.312772 100.839323) (xy 195.259856 100.463606) (xy 195.213554 100.086584)
   (xy 195.176512 99.708227) (xy 195.147408 99.32987) (xy 195.127565 98.951517) (xy 195.115658 98.573164) (xy 195.11169 98.194807)
   (xy 195.116981 97.816454) (xy 195.131533 97.439424) (xy 195.155346 97.062391) (xy 195.187096 96.688009) (xy 195.228106 96.313619)
   (xy 195.278377 95.939237) (xy 195.336585 95.567499) (xy 195.404054 95.198404) (xy 195.47946 94.829309) (xy 195.562804 94.462862)
   (xy 195.655408 94.097734) (xy 195.75595 93.735258) (xy 195.863106 93.374097) (xy 195.979522 93.015588) (xy 196.102554 92.659727)
   (xy 196.233523 92.306509) (xy 196.371106 91.955934) (xy 196.516627 91.608007) (xy 196.670085 91.262724) (xy 196.828835 90.920091)
   (xy 196.995523 90.581423) (xy 197.167502 90.246725) (xy 197.347418 89.914674) (xy 197.53395 89.585268) (xy 197.725772 89.261152)
   (xy 197.92421 88.939684) (xy 198.127939 88.622186) (xy 198.338283 88.307329) (xy 198.553919 87.99777) (xy 198.774845 87.692175)
   (xy 199.001064 87.389227) (xy 199.232575 87.090246) (xy 199.469377 86.796556) (xy 199.711471 86.505518) (xy 199.958856 86.218443)
   (xy 200.21021 85.935342) (xy 200.465532 85.65753) (xy 200.726148 85.38236) (xy 200.99073 85.111162) (xy 201.259282 84.845255)
   (xy 201.531803 84.581995) (xy 201.808293 84.324026) (xy 202.087429 84.070028) (xy 202.371856 83.819994) (xy 202.658929 83.573934)
   (xy 202.948648 83.331838) (xy 203.242335 83.095041) (xy 203.538669 82.863531) (xy 203.83897 82.635988) (xy 204.144564 82.41374)
   (xy 204.452804 82.198103) (xy 204.765012 81.98776) (xy 205.081188 81.784029) (xy 205.402658 81.585592) (xy 205.729418 81.39509)
   (xy 206.060146 81.211202) (xy 206.394844 81.033933) (xy 206.733511 80.861955) (xy 207.073502 80.692621) (xy 207.416136 80.524614)
   (xy 207.758772 80.3566) (xy 208.100084 80.187269) (xy 208.438751 80.013967) (xy 208.774773 79.835371) (xy 209.108147 79.651487)
   (xy 209.434906 79.458337) (xy 209.752407 79.255933) (xy 210.011698 79.032358) (xy 210.146637 78.778364) (xy 210.125469 78.489969)
   (xy 209.983917 78.192312) (xy 209.765637 77.909204) (xy 209.497084 77.641977) (xy 209.192812 77.387975) (xy 208.870022 77.140592)
   (xy 208.545906 76.894529) (xy 208.233698 76.643171) (xy 207.946625 76.383882) (xy 207.682041 76.115331) (xy 207.433334 75.838842)
   (xy 207.199179 75.555734) (xy 206.971636 75.264696) (xy 206.748064 74.969682) (xy 206.52846 74.668058) (xy 206.314146 74.361143)
   (xy 206.106449 74.048937) (xy 205.906689 73.728788) (xy 205.716189 73.403352) (xy 205.534949 73.072622) (xy 205.36297 72.735281)
   (xy 205.201574 72.392645) (xy 205.049439 72.044718) (xy 204.907887 71.692819) (xy 204.776919 71.33563) (xy 204.656532 70.975797)
   (xy 204.545408 70.611997) (xy 204.446189 70.24555) (xy 204.357553 69.876455) (xy 204.279501 69.504717) (xy 204.212032 69.131654)
   (xy 204.15647 68.757269) (xy 204.112814 68.381563) (xy 204.079741 68.00585) (xy 204.058575 67.62882) (xy 204.047991 67.251789)
   (xy 204.050636 66.876081) (xy 204.063867 66.501695) (xy 204.090325 66.128635) (xy 204.128689 65.755571) (xy 204.17896 65.386478)
   (xy 204.241137 65.017383) (xy 204.316543 64.650934) (xy 204.403856 64.28581) (xy 204.503075 63.920686) (xy 204.614199 63.558206)
   (xy 204.73723 63.195726) (xy 204.872168 62.834572) (xy 205.020334 62.473415) (xy 205.179084 62.113582) (xy 205.329898 61.759039)
   (xy 205.410595 61.42831) (xy 205.357679 61.141237) (xy 205.169824 60.913696) (xy 204.874814 60.758915) (xy 204.50572 60.680862)
   (xy 204.107522 60.650436) (xy 203.721231 60.639852) (xy 203.350813 60.627947) (xy 202.977751 60.593549) (xy 202.582199 60.519466)
   (xy 202.173418 60.397758) (xy 201.781836 60.229747) (xy 201.437876 60.016758) (xy 201.171971 59.760112) (xy 201.01322 59.461134)
   (xy 200.961626 59.131727) (xy 201.002636 58.789091) (xy 201.1217 58.450426) (xy 201.304262 58.134248) (xy 201.53445 57.856435)
   (xy 201.800356 57.627571) (xy 202.098012 57.443685) (xy 202.42345 57.302135) (xy 202.772699 57.194977) (xy 203.140471 57.119571)
   (xy 203.524117 57.070625) (xy 203.919668 57.041519) (xy 204.321835 57.02829) (xy 204.72797 57.025644) (xy 205.134106 57.02829)
   (xy 205.534949 57.033582) (xy 205.927855 57.032259) (xy 206.310179 57.016384) (xy 206.679272 56.976696) (xy 207.032492 56.902612)
   (xy 207.368511 56.784874) (xy 207.682041 56.615541) (xy 207.970438 56.402551) (xy 208.227085 56.149873) (xy 208.448012 55.865448)
   (xy 208.627928 55.554561) (xy 208.764189 55.226478) (xy 208.855471 54.882518) (xy 208.907065 54.526655) (xy 208.922939 54.158884)
   (xy 208.909708 53.784498) (xy 208.870022 53.402176) (xy 208.81049 53.017208) (xy 208.733763 52.629593) (xy 208.64645 52.241977)
   (xy 208.551199 51.85701) (xy 208.454626 51.477333) (xy 208.359377 51.102946) (xy 208.264126 50.733852) (xy 208.168877 50.371374)
   (xy 208.072304 50.012863) (xy 207.973086 49.658321) (xy 207.868574 49.306427) (xy 207.758772 48.958499) (xy 207.642357 48.610572)
   (xy 207.516678 48.263967) (xy 207.381741 47.918686) (xy 207.234898 47.572082) (xy 207.080116 47.224155) (xy 206.920042 46.876228)
   (xy 206.756001 46.526978) (xy 206.594605 46.175082) (xy 206.437178 45.82054) (xy 206.289013 45.463353) (xy 206.150105 45.10352)
   (xy 206.028397 44.741041) (xy 205.923887 44.374593) (xy 205.840542 44.004176) (xy 205.783658 43.632436) (xy 205.765136 43.269957)
   (xy 205.796887 42.929968) (xy 205.888169 42.62702) (xy 206.054856 42.370374) (xy 206.299595 42.171937) (xy 206.611803 42.02377)
   (xy 206.97296 41.912645) (xy 207.36719 41.827978) (xy 207.774649 41.760509) (xy 208.180782 41.699655) (xy 208.577658 41.638801)
   (xy 208.967917 41.57927) (xy 209.351565 41.521062) (xy 209.729918 41.464176) (xy 210.10298 41.408613) (xy 210.473396 41.355697)
   (xy 210.841168 41.304103) (xy 211.207617 41.253832) (xy 211.574062 41.204884) (xy 211.940512 41.158582) (xy 212.308281 41.114927)
   (xy 212.677376 41.072592) (xy 213.047794 41.031583) (xy 213.419533 40.993218) (xy 213.792595 40.957499) (xy 214.166979 40.923103)
   (xy 214.541365 40.890031) (xy 214.917072 40.859604) (xy 215.294106 40.831822) (xy 215.671135 40.805364) (xy 216.04949 40.780228)
   (xy 216.427843 40.757739) (xy 216.806198 40.737895) (xy 217.185877 40.719374) (xy 217.565554 40.702176) (xy 217.945229 40.687624)
   (xy 218.324907 40.674395) (xy 218.704584 40.663812) (xy 219.084261 40.655874) (xy 219.46394 40.647937) (xy 219.843615 40.643968)
   (xy 220.223292 40.64) (xy 220.601647 40.638676))
  (stroke (width 0.595312) (type solid)) (fill no) (layer "Edge.Cuts"))
 (gr_arc (start 200 135) (mid 200 135) (end 200 135) (stroke (width 0.05) (type default)) (layer "Edge.Cuts"))
 (segment (start 205.232 90.629288) (end 205.232 102.567288) (width 1) (layer "B.Cu") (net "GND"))
 (segment (start 205.486 97.995288) (end 219.964 97.995288) (width 1) (layer "B.Cu") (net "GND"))
 (segment (start 205.232 97.741288) (end 205.486 97.995288) (width 1) (layer "B.Cu") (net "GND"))
 (segment (start 219.964 84.787288) (end 211.074 84.787288) (width 1) (layer "B.Cu") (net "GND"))
 (segment (start 210.82 71.071288) (end 210.82 72.898) (width 1) (layer "B.Cu") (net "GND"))
 (segment (start 205.232 102.567288) (end 215.9 113.235288) (width 1) (layer "B.Cu") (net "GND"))
 (segment (start 217.018644 79.096644) (end 226.568 69.547288) (width 1) (layer "B.Cu") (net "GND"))
 (segment (start 226.568 69.547288) (end 226.568 68.909288) (width 1) (layer "B.Cu") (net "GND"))
 (segment (start 219.964 82.042) (end 219.964 84.787288) (width 1) (layer "B.Cu") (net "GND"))
 (segment (start 226.568 64.237288) (end 226.568 68.909288) (width 1) (layer "B.Cu") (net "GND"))
 (segment (start 221.537382 85.987288) (end 223.001057 85.987288) (width 0.2) (layer "B.Cu") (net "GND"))
 (segment (start 211.074 84.787288) (end 205.232 90.629288) (width 1) (layer "B.Cu") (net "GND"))
 (segment (start 210.82 72.898) (end 219.964 82.042) (width 1) (layer "B.Cu") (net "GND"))
 (segment (start 226.568 68.909288) (end 228.73 71.071288) (width 1) (layer "B.Cu") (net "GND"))
 (segment (start 215.9 113.235288) (end 219.964 113.235288) (width 1) (layer "B.Cu") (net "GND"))
 (segment (start 222.504 113.235288) (end 230.378 113.235288) (width 1) (layer "B.Cu") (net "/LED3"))
 (segment (start 230.886 105.615288) (end 225.044 105.615288) (width 1) (layer "B.Cu") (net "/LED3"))
 (segment (start 230.378 113.235288) (end 230.886 112.727288) (width 1) (layer "B.Cu") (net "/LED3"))
 (segment (start 230.886 112.727288) (end 230.886 105.615288) (width 1) (layer "B.Cu") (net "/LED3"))
 (segment (start 225.044 82.247288) (end 222.504 84.787288) (width 1) (layer "B.Cu") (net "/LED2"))
 (segment (start 225.044 75.135288) (end 225.044 82.247288) (width 1) (layer "B.Cu") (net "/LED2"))
 (segment (start 217.424 102.567288) (end 217.424 105.615288) (width 1) (layer "B.Cu") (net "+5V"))
 (segment (start 221.996 57.609288) (end 218.313 61.292288) (width 1) (layer "B.Cu") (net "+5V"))
 (segment (start 227.076 57.609288) (end 225.298 57.609288) (width 1) (layer "B.Cu") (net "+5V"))
 (segment (start 231.394 102.567288) (end 217.424 102.567288) (width 1) (layer "B.Cu") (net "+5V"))
 (segment (start 227.584 77.675288) (end 233.426 71.833288) (width 1) (layer "B.Cu") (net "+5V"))
 (segment (start 232.41 97.487288) (end 232.41 101.551288) (width 1) (layer "B.Cu") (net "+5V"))
 (segment (start 232.156 62.689288) (end 227.076 57.609288) (width 1) (layer "B.Cu") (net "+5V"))
 (segment (start 215.9 63.705288) (end 218.313 61.292288) (width 1) (layer "B.Cu") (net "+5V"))
 (segment (start 227.584 89.105288) (end 227.584 77.675288) (width 1) (layer "B.Cu") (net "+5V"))
 (segment (start 218.821 60.784288) (end 221.234 63.197288) (width 1) (layer "B.Cu") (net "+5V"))
 (segment (start 232.41 101.551288) (end 231.394 102.567288) (width 1) (layer "B.Cu") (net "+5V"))
 (segment (start 215.9 64.237288) (end 217.423999 65.761287) (width 1) (layer "B.Cu") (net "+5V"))
 (segment (start 226.568 91.645288) (end 232.41 97.487288) (width 1) (layer "B.Cu") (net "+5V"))
 (segment (start 225.044 91.645288) (end 226.568 91.645288) (width 1) (layer "B.Cu") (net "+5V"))
 (segment (start 232.156 65.991288) (end 232.156 62.689288) (width 1) (layer "B.Cu") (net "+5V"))
 (segment (start 215.9 64.237288) (end 215.9 63.705288) (width 1) (layer "B.Cu") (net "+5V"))
 (segment (start 233.426 67.261288) (end 232.156 65.991288) (width 1) (layer "B.Cu") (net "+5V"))
 (segment (start 225.044 91.645288) (end 227.584 89.105288) (width 1) (layer "B.Cu") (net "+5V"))
 (segment (start 217.423999 65.761287) (end 217.423999 75.135288) (width 1) (layer "B.Cu") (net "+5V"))
 (segment (start 233.426 71.833288) (end 233.426 67.261288) (width 1) (layer "B.Cu") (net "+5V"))
 (segment (start 225.298 57.609288) (end 221.996 57.609288) (width 1) (layer "B.Cu") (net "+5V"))
 (segment (start 217.17 57.101288) (end 216.154 57.101288) (width 1) (layer "B.Cu") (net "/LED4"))
 (segment (start 217.678 57.609288) (end 217.17 57.101288) (width 1) (layer "B.Cu") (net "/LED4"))
 (segment (start 213.36 68.023288) (end 213.36 71.071288) (width 1) (layer "B.Cu") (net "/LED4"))
 (segment (start 211.836 61.419288) (end 211.836 66.499288) (width 1) (layer "B.Cu") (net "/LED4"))
 (segment (start 211.836 66.499288) (end 213.36 68.023288) (width 1) (layer "B.Cu") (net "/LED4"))
 (segment (start 216.154 57.101288) (end 211.836 61.419288) (width 1) (layer "B.Cu") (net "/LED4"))
 (segment (start 226.187 96.598288) (end 224.79 97.995288) (width 1) (layer "B.Cu") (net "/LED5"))
 (segment (start 221.234 91.645288) (end 226.187 96.598288) (width 1) (layer "B.Cu") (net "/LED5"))
 (segment (start 224.79 97.995288) (end 222.504 97.995288) (width 1) (layer "B.Cu") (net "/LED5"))
 (segment (start 217.424 91.645288) (end 221.234 91.645288) (width 1) (layer "B.Cu") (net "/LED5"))
 (segment (start 229.87 63.451288) (end 229.87 66.753288) (width 1) (layer "B.Cu") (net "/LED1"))
 (segment (start 221.234 65.737288) (end 225.552 61.419288) (width 1) (layer "B.Cu") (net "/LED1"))
 (segment (start 227.838 61.419288) (end 229.87 63.451288) (width 1) (layer "B.Cu") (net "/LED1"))
 (segment (start 225.552 61.419288) (end 227.838 61.419288) (width 1) (layer "B.Cu") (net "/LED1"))
 (segment (start 221.234 70.817288) (end 221.234 65.737288) (width 1) (layer "B.Cu") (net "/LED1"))
 (segment (start 229.87 66.753288) (end 231.27 68.153288) (width 1) (layer "B.Cu") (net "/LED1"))
 (segment (start 231.27 68.153288) (end 231.27 71.071288) (width 1) (layer "B.Cu") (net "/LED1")))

